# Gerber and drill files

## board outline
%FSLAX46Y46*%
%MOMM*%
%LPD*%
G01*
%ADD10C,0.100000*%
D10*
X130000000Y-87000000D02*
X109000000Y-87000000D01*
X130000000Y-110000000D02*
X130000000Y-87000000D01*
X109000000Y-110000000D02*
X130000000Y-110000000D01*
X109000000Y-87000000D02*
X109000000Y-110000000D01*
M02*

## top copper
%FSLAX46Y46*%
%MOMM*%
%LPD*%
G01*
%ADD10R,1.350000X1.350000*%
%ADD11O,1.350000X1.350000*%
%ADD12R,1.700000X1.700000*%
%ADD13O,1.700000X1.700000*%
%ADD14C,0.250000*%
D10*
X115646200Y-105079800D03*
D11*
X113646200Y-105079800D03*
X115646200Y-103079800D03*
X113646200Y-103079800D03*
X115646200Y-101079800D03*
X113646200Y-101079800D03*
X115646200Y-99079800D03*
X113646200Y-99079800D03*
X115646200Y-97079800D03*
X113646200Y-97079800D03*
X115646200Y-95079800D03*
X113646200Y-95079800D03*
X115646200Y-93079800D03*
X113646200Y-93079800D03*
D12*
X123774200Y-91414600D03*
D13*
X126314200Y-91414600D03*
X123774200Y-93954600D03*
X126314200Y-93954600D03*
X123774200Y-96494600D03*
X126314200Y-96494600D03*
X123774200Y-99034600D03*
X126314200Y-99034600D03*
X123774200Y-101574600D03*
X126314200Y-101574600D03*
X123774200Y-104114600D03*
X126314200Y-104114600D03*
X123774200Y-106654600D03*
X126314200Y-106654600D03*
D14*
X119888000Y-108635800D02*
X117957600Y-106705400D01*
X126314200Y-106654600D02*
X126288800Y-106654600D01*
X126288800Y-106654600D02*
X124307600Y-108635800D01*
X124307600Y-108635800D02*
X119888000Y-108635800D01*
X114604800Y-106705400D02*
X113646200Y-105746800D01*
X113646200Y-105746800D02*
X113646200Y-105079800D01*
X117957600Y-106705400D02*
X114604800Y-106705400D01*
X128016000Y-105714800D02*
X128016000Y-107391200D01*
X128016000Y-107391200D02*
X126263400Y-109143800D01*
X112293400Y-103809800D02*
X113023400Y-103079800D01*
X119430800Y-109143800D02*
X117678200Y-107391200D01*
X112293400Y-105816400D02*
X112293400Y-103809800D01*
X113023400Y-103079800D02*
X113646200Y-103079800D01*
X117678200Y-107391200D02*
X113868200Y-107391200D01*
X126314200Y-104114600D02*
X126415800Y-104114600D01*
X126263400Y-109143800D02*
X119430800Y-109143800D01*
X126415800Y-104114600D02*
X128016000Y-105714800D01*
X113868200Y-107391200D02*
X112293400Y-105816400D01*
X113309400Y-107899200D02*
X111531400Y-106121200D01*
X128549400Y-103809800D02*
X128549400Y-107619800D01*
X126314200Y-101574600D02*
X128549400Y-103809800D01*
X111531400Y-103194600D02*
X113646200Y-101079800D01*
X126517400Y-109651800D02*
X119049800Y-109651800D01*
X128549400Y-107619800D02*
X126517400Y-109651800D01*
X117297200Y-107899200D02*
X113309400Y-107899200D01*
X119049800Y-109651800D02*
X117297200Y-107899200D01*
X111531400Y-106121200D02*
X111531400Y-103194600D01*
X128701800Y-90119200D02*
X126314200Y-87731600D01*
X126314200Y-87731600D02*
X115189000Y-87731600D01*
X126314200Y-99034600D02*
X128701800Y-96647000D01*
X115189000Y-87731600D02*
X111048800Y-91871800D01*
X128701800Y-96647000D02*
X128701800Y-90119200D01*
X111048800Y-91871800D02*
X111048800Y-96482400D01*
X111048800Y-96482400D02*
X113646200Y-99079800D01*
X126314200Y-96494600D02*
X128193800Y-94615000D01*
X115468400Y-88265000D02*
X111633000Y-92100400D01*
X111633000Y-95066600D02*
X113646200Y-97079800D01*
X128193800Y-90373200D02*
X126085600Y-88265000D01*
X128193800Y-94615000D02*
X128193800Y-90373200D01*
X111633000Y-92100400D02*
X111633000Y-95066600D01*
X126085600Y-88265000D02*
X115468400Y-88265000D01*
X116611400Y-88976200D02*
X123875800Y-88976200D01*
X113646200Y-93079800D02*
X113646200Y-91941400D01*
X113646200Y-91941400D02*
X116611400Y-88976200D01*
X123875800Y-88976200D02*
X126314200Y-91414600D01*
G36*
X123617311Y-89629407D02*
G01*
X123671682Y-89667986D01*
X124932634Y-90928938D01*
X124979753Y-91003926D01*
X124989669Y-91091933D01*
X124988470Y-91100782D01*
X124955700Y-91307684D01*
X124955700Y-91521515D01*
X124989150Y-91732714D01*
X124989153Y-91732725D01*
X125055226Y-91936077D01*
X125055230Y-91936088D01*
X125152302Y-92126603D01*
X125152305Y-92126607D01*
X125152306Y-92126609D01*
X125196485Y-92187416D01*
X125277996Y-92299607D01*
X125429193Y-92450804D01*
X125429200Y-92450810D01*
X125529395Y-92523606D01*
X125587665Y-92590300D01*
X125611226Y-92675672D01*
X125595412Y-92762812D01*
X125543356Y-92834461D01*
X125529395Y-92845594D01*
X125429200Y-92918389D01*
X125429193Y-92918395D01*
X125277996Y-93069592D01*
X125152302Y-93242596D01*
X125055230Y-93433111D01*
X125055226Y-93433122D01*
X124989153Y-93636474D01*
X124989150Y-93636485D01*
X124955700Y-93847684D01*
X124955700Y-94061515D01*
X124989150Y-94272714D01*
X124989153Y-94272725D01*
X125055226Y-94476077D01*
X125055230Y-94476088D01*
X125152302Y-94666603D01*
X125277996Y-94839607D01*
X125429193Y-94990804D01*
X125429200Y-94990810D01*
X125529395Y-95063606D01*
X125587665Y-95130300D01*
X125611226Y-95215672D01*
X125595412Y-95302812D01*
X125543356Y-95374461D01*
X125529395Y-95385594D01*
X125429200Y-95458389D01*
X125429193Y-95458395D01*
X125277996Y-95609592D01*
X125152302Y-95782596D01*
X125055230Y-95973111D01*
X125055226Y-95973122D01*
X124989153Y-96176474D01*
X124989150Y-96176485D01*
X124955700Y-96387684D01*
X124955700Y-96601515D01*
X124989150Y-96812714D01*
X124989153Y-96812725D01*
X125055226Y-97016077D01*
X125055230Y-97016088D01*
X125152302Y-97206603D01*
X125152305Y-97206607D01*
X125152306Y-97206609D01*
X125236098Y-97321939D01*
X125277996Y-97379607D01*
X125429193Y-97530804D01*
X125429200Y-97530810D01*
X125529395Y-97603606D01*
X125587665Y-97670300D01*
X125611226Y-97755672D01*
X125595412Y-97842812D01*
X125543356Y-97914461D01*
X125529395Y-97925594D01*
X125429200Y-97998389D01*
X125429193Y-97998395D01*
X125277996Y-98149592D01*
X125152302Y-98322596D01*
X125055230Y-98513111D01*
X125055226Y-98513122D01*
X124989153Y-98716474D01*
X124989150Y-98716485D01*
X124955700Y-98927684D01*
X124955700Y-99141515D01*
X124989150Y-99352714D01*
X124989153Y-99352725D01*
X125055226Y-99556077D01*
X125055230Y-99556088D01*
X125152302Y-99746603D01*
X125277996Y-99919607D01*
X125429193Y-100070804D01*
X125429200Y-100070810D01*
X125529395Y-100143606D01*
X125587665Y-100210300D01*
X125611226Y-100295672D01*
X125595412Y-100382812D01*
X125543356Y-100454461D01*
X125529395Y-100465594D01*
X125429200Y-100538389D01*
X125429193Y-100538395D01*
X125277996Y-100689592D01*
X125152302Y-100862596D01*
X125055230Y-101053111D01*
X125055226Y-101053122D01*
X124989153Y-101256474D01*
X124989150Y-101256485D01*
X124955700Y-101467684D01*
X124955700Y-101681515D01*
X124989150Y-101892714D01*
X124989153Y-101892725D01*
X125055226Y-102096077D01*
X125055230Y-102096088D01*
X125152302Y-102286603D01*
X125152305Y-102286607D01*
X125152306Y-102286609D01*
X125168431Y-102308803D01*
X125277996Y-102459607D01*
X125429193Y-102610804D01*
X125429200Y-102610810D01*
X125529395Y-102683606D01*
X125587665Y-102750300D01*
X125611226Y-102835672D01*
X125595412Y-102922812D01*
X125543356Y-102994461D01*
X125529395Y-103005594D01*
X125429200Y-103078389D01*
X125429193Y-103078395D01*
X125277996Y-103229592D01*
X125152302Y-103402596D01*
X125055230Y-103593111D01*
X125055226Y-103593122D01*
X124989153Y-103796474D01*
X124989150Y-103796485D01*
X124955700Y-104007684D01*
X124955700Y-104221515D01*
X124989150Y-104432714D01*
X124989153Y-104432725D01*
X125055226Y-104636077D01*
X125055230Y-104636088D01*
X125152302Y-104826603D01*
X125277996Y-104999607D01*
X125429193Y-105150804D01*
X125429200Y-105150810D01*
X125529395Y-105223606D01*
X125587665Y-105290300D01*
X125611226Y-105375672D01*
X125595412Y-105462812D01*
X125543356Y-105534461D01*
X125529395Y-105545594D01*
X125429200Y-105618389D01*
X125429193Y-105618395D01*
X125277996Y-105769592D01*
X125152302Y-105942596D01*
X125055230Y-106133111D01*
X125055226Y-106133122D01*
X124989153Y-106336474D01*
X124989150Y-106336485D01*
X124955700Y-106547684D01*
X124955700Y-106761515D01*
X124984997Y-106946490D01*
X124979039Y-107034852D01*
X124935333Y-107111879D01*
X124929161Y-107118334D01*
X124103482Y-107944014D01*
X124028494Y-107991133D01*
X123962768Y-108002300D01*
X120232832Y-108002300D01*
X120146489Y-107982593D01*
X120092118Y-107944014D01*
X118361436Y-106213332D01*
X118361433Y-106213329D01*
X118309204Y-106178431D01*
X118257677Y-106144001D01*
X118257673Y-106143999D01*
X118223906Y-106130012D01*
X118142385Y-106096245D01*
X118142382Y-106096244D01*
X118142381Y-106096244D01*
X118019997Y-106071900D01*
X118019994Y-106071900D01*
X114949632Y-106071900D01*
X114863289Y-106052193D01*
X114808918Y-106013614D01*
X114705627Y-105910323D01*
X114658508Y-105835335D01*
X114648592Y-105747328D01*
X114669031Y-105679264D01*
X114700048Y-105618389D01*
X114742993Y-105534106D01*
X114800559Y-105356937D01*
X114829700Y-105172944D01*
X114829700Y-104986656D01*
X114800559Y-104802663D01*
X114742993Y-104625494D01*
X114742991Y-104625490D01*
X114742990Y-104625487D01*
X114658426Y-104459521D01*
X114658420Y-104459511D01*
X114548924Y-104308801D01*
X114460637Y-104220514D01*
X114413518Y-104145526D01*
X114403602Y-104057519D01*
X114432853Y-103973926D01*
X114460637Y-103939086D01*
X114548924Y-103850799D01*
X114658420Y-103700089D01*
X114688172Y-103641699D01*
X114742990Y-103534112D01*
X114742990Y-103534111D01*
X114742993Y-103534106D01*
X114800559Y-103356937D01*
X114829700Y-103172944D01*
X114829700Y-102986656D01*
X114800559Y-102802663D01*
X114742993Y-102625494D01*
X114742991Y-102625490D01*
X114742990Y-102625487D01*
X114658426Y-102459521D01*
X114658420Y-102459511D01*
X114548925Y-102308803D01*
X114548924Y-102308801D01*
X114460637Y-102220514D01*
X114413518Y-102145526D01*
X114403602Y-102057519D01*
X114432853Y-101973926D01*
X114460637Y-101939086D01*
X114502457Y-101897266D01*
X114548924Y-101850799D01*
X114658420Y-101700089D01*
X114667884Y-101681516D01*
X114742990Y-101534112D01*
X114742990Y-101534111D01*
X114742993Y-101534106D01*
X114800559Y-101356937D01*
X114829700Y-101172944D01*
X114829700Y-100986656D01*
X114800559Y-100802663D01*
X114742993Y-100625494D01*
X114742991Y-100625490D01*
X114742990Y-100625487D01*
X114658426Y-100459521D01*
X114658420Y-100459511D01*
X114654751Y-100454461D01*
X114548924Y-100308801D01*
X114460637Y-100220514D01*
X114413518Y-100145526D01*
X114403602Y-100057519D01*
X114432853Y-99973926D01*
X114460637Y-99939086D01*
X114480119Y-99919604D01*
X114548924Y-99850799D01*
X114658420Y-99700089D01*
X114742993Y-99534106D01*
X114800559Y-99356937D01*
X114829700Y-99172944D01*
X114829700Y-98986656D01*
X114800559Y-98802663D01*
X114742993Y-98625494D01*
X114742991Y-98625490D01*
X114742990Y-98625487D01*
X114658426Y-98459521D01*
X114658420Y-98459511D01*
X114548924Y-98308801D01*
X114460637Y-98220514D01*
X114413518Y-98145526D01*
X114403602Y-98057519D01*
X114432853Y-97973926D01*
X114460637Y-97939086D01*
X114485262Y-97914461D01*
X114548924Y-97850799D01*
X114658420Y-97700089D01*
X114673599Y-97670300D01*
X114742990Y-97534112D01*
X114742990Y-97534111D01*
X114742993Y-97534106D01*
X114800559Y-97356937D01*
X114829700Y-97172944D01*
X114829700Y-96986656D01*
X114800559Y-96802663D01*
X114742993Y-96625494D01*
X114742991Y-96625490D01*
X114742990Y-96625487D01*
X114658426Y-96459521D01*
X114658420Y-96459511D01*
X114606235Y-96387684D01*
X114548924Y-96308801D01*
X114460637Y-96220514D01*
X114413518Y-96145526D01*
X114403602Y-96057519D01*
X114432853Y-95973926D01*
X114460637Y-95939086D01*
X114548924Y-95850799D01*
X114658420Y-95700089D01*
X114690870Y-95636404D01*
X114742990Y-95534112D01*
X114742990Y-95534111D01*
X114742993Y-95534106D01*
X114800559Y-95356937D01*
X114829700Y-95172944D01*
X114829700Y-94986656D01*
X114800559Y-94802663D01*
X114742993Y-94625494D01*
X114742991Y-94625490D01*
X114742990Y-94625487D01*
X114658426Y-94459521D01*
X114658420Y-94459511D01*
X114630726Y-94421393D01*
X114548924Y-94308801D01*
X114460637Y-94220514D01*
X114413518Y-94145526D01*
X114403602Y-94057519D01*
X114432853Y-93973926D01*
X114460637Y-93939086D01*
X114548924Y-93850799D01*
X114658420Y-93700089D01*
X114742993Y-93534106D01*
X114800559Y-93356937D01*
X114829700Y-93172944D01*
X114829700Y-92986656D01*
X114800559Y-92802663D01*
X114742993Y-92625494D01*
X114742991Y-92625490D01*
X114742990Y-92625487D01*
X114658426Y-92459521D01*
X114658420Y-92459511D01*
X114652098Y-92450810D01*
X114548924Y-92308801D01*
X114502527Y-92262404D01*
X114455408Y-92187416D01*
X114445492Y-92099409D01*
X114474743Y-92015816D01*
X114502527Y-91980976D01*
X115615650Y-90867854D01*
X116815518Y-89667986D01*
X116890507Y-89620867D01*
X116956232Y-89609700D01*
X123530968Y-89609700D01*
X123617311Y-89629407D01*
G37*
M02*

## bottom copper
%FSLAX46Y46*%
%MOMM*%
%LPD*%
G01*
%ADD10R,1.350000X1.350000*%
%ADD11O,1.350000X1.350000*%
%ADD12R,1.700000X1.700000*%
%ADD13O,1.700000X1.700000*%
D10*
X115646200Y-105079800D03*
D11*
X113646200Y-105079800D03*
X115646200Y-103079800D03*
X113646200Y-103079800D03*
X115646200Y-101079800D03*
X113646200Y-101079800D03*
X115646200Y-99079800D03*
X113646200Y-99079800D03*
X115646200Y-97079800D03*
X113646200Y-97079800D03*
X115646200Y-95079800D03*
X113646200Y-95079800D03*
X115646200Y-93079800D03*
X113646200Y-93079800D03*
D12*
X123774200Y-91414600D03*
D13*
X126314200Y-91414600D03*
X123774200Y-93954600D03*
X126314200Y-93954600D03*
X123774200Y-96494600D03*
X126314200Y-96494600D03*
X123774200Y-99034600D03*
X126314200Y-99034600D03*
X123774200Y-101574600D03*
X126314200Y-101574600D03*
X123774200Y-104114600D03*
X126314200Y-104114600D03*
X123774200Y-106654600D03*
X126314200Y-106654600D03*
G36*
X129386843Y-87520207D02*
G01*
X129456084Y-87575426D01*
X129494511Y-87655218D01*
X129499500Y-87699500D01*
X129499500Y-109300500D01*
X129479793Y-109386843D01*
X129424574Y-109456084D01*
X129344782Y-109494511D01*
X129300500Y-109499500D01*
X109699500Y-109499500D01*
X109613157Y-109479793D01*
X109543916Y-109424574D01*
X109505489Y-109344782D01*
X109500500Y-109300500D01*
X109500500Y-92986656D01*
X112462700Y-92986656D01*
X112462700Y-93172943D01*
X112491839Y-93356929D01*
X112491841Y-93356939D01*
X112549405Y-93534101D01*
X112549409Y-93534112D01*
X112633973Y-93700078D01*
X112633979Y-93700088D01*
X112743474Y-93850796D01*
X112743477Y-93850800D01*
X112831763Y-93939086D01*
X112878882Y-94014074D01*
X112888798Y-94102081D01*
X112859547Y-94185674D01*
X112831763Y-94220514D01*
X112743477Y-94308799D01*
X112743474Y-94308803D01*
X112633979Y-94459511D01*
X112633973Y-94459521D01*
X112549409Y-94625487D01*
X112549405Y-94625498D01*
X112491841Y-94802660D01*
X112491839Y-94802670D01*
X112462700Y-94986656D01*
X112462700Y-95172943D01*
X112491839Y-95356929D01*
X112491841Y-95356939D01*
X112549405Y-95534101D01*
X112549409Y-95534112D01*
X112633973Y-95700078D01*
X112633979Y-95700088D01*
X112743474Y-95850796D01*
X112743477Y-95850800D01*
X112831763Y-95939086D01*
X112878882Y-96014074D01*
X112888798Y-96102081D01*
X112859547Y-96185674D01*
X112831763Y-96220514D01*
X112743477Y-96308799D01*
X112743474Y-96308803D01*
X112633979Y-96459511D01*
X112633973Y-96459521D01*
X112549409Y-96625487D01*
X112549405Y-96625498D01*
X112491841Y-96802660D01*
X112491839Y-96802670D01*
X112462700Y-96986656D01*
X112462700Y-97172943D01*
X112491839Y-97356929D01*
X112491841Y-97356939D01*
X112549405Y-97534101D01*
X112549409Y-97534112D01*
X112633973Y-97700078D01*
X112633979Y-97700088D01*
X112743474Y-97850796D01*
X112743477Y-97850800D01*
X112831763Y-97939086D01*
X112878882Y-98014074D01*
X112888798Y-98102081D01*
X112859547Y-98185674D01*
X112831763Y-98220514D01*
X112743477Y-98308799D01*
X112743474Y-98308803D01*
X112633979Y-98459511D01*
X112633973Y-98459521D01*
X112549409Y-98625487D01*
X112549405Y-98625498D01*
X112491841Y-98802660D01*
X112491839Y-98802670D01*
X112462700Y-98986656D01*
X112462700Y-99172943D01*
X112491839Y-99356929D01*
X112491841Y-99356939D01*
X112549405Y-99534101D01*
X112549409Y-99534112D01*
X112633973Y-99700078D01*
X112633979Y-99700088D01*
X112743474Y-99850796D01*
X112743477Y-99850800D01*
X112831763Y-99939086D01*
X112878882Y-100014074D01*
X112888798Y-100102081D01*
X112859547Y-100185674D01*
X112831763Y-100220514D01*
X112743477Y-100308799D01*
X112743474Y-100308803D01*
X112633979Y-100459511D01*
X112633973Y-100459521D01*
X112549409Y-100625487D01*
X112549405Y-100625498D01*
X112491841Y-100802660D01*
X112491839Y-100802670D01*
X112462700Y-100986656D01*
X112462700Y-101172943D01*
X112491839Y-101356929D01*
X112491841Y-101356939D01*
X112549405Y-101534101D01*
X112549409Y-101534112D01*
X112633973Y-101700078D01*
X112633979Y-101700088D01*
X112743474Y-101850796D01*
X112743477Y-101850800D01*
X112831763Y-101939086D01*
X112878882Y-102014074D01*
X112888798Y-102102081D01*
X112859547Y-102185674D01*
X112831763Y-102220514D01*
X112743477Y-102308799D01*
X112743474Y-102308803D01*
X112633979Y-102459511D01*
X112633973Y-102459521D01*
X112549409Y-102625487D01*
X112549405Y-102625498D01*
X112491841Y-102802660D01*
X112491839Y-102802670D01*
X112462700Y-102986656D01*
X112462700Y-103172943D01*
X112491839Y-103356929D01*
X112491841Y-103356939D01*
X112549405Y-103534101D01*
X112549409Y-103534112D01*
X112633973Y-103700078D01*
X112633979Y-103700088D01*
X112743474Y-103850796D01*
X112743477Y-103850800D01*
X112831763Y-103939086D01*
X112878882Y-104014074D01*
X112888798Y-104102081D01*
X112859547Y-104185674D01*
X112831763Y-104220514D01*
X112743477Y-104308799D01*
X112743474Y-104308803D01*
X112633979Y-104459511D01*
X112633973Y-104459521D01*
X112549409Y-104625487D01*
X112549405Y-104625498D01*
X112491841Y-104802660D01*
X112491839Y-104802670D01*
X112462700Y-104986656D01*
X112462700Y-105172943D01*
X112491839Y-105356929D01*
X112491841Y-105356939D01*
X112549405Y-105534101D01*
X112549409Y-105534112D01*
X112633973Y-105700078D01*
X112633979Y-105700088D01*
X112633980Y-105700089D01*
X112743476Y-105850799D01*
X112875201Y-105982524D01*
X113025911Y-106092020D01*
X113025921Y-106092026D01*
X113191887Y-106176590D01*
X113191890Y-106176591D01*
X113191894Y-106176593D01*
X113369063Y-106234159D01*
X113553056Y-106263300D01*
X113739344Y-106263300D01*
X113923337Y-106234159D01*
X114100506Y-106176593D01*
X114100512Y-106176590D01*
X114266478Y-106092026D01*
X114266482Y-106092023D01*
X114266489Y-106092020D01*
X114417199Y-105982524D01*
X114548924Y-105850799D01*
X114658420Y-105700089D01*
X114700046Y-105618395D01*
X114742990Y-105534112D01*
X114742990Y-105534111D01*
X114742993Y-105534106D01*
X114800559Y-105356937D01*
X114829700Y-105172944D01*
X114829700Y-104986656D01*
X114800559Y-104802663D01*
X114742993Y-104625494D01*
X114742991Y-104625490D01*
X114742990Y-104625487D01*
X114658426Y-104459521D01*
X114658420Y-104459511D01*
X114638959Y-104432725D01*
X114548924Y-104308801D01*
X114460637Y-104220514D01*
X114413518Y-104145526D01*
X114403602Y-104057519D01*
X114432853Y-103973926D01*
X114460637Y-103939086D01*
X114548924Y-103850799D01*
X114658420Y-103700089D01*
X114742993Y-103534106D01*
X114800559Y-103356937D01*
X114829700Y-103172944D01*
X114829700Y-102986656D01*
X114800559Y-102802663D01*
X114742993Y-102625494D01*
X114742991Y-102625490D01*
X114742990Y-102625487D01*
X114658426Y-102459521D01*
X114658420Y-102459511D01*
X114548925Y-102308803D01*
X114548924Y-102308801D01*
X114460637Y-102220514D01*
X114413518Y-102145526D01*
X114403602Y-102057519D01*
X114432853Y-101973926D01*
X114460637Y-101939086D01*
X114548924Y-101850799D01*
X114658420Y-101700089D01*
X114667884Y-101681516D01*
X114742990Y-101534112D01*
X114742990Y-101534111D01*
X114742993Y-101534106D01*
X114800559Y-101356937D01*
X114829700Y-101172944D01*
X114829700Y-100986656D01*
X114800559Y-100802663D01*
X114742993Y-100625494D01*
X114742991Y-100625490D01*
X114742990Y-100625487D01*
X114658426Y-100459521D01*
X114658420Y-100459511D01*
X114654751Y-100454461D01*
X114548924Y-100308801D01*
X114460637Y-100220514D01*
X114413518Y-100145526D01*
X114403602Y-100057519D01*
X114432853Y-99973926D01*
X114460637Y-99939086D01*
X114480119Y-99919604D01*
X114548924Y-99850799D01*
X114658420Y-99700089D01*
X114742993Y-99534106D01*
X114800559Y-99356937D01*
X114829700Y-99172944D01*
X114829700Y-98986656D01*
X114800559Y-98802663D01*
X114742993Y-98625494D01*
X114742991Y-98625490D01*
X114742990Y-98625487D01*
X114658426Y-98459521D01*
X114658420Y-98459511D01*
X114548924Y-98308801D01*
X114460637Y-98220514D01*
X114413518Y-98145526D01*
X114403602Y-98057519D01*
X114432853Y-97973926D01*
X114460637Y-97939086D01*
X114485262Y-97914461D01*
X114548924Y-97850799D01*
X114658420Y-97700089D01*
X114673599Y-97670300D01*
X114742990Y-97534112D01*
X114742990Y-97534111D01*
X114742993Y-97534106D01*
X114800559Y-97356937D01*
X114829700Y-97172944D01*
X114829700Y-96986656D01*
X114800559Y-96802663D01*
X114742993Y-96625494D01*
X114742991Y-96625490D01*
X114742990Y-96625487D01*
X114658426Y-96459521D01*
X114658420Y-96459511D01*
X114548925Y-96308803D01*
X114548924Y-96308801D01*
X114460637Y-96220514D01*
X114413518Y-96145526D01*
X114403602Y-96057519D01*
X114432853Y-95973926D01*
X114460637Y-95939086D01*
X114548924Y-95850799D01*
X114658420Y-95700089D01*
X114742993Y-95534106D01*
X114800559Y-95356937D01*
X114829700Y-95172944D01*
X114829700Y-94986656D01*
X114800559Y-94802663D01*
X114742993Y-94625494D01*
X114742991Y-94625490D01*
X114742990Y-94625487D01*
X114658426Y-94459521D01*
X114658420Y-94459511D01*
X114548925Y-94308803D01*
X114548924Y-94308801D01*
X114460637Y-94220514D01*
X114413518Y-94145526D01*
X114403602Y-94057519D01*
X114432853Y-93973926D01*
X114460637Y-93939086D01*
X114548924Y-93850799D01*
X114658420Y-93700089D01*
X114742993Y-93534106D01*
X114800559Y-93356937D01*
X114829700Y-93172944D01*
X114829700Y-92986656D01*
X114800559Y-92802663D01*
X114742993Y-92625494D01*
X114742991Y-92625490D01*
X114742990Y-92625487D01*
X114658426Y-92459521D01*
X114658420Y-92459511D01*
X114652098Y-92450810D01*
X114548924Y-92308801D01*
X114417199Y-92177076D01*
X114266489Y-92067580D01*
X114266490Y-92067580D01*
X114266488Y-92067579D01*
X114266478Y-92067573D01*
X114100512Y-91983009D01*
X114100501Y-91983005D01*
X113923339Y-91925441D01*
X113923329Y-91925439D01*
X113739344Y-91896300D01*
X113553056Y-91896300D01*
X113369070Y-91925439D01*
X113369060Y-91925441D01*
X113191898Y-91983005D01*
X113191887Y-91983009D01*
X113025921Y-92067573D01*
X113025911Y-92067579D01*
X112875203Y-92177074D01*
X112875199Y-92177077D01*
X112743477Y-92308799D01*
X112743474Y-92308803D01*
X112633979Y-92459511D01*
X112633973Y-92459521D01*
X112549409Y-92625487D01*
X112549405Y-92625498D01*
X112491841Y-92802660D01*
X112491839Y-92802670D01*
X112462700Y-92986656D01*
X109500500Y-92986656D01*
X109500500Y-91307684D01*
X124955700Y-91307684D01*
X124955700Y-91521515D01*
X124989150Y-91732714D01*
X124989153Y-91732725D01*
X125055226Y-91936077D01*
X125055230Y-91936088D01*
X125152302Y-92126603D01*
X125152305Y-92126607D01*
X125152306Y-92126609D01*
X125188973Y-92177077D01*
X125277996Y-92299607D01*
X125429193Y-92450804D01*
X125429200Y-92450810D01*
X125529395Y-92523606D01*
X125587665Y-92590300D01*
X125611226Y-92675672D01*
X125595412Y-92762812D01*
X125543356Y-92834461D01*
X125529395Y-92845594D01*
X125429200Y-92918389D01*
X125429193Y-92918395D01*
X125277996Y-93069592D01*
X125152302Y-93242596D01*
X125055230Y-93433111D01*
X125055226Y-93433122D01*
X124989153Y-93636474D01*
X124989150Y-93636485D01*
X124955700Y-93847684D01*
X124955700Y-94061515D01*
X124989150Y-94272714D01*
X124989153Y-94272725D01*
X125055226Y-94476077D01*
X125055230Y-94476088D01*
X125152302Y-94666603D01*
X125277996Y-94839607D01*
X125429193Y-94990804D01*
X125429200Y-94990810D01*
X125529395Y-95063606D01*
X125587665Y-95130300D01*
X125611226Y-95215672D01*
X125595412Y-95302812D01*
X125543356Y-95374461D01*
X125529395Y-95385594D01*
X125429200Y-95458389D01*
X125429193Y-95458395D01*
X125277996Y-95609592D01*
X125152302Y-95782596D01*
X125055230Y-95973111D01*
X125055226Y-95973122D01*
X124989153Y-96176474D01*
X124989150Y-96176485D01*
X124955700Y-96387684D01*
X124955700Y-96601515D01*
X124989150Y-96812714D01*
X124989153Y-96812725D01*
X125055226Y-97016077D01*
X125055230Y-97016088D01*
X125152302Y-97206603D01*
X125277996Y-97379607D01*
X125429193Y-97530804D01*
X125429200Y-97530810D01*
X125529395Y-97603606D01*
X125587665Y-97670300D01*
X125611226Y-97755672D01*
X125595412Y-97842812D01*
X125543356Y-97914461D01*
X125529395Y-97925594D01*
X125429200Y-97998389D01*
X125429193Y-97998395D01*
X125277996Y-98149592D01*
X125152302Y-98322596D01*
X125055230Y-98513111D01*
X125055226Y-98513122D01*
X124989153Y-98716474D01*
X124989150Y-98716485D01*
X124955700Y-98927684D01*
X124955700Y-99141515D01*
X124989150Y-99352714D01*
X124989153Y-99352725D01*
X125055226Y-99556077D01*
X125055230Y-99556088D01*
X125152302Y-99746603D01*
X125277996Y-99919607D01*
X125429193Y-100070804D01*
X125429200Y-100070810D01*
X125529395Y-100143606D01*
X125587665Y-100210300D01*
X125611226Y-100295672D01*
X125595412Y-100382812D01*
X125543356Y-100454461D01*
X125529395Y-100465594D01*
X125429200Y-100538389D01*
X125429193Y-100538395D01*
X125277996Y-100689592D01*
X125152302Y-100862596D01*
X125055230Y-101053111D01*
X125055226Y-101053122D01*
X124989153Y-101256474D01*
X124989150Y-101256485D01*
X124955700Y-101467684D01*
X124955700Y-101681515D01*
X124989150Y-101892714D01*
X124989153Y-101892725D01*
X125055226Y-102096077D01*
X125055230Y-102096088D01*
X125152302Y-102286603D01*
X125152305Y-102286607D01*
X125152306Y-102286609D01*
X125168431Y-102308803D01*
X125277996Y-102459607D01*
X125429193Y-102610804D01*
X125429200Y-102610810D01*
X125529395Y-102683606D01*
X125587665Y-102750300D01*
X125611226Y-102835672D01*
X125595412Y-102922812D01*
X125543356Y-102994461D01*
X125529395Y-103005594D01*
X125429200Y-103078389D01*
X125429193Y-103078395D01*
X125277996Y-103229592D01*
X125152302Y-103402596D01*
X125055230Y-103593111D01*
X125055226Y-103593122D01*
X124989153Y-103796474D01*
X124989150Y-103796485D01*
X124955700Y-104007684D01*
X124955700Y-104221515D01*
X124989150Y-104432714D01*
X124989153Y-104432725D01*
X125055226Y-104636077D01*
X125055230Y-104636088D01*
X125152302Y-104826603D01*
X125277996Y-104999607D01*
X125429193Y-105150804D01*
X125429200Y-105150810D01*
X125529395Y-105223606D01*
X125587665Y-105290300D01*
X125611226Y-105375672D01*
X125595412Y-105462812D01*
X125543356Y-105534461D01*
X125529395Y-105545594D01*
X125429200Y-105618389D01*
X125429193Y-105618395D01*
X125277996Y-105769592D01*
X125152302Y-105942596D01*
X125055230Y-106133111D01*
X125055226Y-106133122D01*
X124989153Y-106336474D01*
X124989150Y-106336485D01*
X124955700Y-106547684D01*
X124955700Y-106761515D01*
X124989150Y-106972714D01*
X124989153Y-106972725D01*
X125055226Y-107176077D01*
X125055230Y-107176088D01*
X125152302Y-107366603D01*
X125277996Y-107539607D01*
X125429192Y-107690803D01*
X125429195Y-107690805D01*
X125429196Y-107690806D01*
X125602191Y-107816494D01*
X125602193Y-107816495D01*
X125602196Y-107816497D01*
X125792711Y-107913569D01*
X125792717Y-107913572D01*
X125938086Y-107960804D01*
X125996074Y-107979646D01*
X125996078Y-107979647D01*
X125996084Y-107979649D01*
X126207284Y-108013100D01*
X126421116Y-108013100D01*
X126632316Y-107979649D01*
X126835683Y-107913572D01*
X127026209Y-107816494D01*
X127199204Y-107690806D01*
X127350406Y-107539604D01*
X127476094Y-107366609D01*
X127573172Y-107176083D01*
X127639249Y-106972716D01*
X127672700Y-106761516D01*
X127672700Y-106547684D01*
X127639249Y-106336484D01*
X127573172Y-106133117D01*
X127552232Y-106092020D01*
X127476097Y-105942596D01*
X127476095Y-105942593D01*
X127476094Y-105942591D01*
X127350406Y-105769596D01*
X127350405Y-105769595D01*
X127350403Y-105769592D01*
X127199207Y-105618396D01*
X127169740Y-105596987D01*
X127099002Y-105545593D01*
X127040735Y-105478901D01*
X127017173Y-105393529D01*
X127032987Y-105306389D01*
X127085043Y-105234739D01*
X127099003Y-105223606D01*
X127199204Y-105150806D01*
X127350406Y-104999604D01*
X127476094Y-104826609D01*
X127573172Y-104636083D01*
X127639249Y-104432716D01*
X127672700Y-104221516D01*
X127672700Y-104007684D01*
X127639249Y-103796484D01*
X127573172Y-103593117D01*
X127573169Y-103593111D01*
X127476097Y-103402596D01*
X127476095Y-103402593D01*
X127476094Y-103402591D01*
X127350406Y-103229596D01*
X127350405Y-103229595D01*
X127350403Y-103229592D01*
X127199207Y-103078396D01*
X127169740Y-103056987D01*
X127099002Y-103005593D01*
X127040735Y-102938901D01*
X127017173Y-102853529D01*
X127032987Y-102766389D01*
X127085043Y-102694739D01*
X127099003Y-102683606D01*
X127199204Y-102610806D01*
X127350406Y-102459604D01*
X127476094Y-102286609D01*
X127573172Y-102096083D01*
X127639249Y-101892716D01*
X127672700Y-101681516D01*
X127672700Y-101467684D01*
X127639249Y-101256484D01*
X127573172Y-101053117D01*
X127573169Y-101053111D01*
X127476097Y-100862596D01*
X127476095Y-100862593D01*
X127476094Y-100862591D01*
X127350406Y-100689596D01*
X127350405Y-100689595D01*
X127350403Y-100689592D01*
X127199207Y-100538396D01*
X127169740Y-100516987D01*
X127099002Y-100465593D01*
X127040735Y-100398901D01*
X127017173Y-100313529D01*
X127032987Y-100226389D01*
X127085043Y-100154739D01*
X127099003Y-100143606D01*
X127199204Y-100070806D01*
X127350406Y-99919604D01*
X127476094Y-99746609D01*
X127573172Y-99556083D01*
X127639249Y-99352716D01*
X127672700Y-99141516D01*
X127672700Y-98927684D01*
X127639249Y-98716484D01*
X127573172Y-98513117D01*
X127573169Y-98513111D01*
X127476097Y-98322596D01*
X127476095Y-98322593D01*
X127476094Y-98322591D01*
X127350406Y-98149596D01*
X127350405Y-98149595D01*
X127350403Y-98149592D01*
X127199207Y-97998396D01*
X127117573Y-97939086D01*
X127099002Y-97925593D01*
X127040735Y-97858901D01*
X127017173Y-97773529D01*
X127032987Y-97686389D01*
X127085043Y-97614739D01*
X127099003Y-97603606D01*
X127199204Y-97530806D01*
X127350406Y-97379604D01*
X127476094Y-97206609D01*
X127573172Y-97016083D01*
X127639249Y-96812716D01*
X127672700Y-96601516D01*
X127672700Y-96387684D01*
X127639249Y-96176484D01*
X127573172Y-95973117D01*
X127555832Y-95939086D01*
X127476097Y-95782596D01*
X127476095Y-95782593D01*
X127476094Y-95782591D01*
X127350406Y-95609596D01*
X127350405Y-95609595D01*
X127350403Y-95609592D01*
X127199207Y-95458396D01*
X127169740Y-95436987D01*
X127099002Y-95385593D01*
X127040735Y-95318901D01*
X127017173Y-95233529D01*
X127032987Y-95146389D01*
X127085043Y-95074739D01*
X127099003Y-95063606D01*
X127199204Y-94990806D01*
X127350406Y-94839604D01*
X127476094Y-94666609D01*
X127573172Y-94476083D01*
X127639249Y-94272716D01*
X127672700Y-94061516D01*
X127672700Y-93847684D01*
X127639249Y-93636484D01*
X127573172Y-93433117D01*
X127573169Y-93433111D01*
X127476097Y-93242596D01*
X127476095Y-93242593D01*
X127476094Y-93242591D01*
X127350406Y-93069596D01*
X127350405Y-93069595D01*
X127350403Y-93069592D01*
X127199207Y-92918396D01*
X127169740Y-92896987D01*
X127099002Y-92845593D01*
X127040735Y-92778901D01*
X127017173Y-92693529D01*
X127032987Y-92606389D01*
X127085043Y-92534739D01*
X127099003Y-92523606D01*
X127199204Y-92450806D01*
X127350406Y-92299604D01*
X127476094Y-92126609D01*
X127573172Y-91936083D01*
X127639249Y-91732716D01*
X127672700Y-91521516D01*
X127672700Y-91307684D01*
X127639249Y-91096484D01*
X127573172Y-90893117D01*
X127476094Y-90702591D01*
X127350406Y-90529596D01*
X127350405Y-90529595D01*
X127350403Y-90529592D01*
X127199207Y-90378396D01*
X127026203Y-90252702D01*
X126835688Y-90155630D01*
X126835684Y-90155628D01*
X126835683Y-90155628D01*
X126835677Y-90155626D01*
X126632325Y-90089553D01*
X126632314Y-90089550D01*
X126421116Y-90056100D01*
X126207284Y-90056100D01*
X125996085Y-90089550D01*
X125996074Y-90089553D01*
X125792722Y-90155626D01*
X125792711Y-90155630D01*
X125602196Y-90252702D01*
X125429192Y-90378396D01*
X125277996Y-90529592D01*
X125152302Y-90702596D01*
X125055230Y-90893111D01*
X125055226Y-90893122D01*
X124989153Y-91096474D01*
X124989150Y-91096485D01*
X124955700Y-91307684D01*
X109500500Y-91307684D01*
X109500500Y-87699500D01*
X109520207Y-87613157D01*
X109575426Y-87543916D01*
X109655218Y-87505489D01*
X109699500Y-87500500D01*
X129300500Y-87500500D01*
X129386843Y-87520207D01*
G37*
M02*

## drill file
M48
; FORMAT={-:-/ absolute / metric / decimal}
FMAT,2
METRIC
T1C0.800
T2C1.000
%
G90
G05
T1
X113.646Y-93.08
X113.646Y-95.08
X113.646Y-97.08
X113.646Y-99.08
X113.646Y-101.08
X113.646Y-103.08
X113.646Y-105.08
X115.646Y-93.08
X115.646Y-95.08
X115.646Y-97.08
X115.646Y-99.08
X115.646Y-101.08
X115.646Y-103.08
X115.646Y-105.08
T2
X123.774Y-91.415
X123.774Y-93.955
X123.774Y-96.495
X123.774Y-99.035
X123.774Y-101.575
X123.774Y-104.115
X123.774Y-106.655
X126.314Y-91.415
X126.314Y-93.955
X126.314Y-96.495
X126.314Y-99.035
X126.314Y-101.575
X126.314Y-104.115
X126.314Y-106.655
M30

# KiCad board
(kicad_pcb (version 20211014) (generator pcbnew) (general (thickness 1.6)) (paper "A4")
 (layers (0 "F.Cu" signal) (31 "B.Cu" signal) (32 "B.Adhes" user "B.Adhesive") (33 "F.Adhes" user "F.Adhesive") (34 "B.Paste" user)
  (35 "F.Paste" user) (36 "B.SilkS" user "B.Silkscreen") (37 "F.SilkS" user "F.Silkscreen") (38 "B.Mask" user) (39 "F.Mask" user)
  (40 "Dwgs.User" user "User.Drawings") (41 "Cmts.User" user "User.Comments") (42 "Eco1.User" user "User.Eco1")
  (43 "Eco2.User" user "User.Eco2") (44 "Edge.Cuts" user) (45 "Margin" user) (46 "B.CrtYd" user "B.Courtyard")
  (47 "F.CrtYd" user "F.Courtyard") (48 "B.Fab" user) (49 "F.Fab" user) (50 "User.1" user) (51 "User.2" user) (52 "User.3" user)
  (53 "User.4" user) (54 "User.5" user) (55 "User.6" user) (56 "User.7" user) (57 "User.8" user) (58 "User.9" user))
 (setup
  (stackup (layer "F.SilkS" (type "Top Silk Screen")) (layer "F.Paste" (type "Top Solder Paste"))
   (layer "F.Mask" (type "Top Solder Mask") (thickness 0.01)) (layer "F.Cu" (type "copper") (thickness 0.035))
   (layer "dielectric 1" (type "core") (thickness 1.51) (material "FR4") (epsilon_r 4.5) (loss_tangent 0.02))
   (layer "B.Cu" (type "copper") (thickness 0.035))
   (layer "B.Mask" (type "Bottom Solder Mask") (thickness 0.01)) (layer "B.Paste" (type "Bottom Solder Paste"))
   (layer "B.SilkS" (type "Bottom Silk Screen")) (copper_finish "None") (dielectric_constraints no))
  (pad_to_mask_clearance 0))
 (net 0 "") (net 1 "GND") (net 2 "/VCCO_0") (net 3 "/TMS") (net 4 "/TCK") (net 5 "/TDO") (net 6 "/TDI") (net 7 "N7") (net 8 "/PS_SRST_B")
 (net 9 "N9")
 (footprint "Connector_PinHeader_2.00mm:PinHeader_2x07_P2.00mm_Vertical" (layer "F.Cu") (at 115.6462 105.0798 180)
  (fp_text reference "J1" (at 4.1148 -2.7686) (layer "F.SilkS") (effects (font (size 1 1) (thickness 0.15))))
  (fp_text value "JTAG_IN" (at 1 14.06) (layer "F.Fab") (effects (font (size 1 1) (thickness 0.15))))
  (pad "1" thru_hole rect (at 0 0 180) (size 1.35 1.35) (drill 0.8) (layers *.Cu *.Mask) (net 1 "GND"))
  (pad "2" thru_hole oval (at 2 0 180) (size 1.35 1.35) (drill 0.8) (layers *.Cu *.Mask) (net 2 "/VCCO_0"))
  (pad "3" thru_hole oval (at 0 2 180) (size 1.35 1.35) (drill 0.8) (layers *.Cu *.Mask) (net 1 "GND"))
  (pad "4" thru_hole oval (at 2 2 180) (size 1.35 1.35) (drill 0.8) (layers *.Cu *.Mask) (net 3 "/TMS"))
  (pad "5" thru_hole oval (at 0 4 180) (size 1.35 1.35) (drill 0.8) (layers *.Cu *.Mask) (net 1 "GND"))
  (pad "6" thru_hole oval (at 2 4 180) (size 1.35 1.35) (drill 0.8) (layers *.Cu *.Mask) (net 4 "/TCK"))
  (pad "7" thru_hole oval (at 0 6 180) (size 1.35 1.35) (drill 0.8) (layers *.Cu *.Mask) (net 1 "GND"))
  (pad "8" thru_hole oval (at 2 6 180) (size 1.35 1.35) (drill 0.8) (layers *.Cu *.Mask) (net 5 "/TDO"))
  (pad "9" thru_hole oval (at 0 8 180) (size 1.35 1.35) (drill 0.8) (layers *.Cu *.Mask) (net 1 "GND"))
  (pad "10" thru_hole oval (at 2 8 180) (size 1.35 1.35) (drill 0.8) (layers *.Cu *.Mask) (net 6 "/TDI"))
  (pad "11" thru_hole oval (at 0 10 180) (size 1.35 1.35) (drill 0.8) (layers *.Cu *.Mask) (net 1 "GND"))
  (pad "12" thru_hole oval (at 2 10 180) (size 1.35 1.35) (drill 0.8) (layers *.Cu *.Mask) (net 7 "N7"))
  (pad "13" thru_hole oval (at 0 12 180) (size 1.35 1.35) (drill 0.8) (layers *.Cu *.Mask) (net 1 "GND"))
  (pad "14" thru_hole oval (at 2 12 180) (size 1.35 1.35) (drill 0.8) (layers *.Cu *.Mask) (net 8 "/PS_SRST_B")))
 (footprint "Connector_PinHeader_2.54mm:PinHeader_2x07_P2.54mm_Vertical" (layer "F.Cu") (at 123.7742 91.4146)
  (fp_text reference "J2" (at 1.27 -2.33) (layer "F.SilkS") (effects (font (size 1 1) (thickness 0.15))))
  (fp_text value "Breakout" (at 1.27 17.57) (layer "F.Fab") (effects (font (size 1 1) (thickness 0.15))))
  (pad "1" thru_hole rect (at 0 0) (size 1.7 1.7) (drill 1) (layers *.Cu *.Mask) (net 1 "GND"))
  (pad "2" thru_hole oval (at 2.54 0) (size 1.7 1.7) (drill 1) (layers *.Cu *.Mask) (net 8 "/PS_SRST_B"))
  (pad "3" thru_hole oval (at 0 2.54) (size 1.7 1.7) (drill 1) (layers *.Cu *.Mask) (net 1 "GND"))
  (pad "4" thru_hole oval (at 2.54 2.54) (size 1.7 1.7) (drill 1) (layers *.Cu *.Mask) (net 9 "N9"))
  (pad "5" thru_hole oval (at 0 5.08) (size 1.7 1.7) (drill 1) (layers *.Cu *.Mask) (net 1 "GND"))
  (pad "6" thru_hole oval (at 2.54 5.08) (size 1.7 1.7) (drill 1) (layers *.Cu *.Mask) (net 6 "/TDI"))
  (pad "7" thru_hole oval (at 0 7.62) (size 1.7 1.7) (drill 1) (layers *.Cu *.Mask) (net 1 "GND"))
  (pad "8" thru_hole oval (at 2.54 7.62) (size 1.7 1.7) (drill 1) (layers *.Cu *.Mask) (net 5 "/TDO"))
  (pad "9" thru_hole oval (at 0 10.16) (size 1.7 1.7) (drill 1) (layers *.Cu *.Mask) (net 1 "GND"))
  (pad "10" thru_hole oval (at 2.54 10.16) (size 1.7 1.7) (drill 1) (layers *.Cu *.Mask) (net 4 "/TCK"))
  (pad "11" thru_hole oval (at 0 12.7) (size 1.7 1.7) (drill 1) (layers *.Cu *.Mask) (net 1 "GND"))
  (pad "12" thru_hole oval (at 2.54 12.7) (size 1.7 1.7) (drill 1) (layers *.Cu *.Mask) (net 3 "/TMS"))
  (pad "13" thru_hole oval (at 0 15.24) (size 1.7 1.7) (drill 1) (layers *.Cu *.Mask) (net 1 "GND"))
  (pad "14" thru_hole oval (at 2.54 15.24) (size 1.7 1.7) (drill 1) (layers *.Cu *.Mask) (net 2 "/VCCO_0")))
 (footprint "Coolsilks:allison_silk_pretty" (layer "B.Cu") (at 119.507 104.7496 180)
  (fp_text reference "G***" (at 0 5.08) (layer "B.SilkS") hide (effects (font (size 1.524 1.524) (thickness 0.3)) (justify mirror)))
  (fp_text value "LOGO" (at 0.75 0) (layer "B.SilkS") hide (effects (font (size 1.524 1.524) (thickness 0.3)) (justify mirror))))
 (gr_line (start 130 87) (end 109 87) (layer "Edge.Cuts") (width 0.1))
 (gr_line (start 130 110) (end 130 87) (layer "Edge.Cuts") (width 0.1))
 (gr_line (start 109 110) (end 130 110) (layer "Edge.Cuts") (width 0.1))
 (gr_line (start 109 87) (end 109 110) (layer "Edge.Cuts") (width 0.1))
 (segment (start 119.888 108.6358) (end 117.9576 106.7054) (width 0.25) (layer "F.Cu") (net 2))
 (segment (start 126.3142 106.6546) (end 126.2888 106.6546) (width 0.25) (layer "F.Cu") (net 2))
 (segment (start 126.2888 106.6546) (end 124.3076 108.6358) (width 0.25) (layer "F.Cu") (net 2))
 (segment (start 124.3076 108.6358) (end 119.888 108.6358) (width 0.25) (layer "F.Cu") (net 2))
 (segment (start 114.6048 106.7054) (end 113.6462 105.7468) (width 0.25) (layer "F.Cu") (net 2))
 (segment (start 113.6462 105.7468) (end 113.6462 105.0798) (width 0.25) (layer "F.Cu") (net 2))
 (segment (start 117.9576 106.7054) (end 114.6048 106.7054) (width 0.25) (layer "F.Cu") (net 2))
 (segment (start 128.016 105.7148) (end 128.016 107.3912) (width 0.25) (layer "F.Cu") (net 3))
 (segment (start 128.016 107.3912) (end 126.2634 109.1438) (width 0.25) (layer "F.Cu") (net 3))
 (segment (start 112.2934 103.8098) (end 113.0234 103.0798) (width 0.25) (layer "F.Cu") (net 3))
 (segment (start 119.4308 109.1438) (end 117.6782 107.3912) (width 0.25) (layer "F.Cu") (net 3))
 (segment (start 112.2934 105.8164) (end 112.2934 103.8098) (width 0.25) (layer "F.Cu") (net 3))
 (segment (start 113.0234 103.0798) (end 113.6462 103.0798) (width 0.25) (layer "F.Cu") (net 3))
 (segment (start 117.6782 107.3912) (end 113.8682 107.3912) (width 0.25) (layer "F.Cu") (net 3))
 (segment (start 126.3142 104.1146) (end 126.4158 104.1146) (width 0.25) (layer "F.Cu") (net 3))
 (segment (start 126.2634 109.1438) (end 119.4308 109.1438) (width 0.25) (layer "F.Cu") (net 3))
 (segment (start 126.4158 104.1146) (end 128.016 105.7148) (width 0.25) (layer "F.Cu") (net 3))
 (segment (start 113.8682 107.3912) (end 112.2934 105.8164) (width 0.25) (layer "F.Cu") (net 3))
 (segment (start 113.3094 107.8992) (end 111.5314 106.1212) (width 0.25) (layer "F.Cu") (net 4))
 (segment (start 128.5494 103.8098) (end 128.5494 107.6198) (width 0.25) (layer "F.Cu") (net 4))
 (segment (start 126.3142 101.5746) (end 128.5494 103.8098) (width 0.25) (layer "F.Cu") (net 4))
 (segment (start 111.5314 103.1946) (end 113.6462 101.0798) (width 0.25) (layer "F.Cu") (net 4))
 (segment (start 126.5174 109.6518) (end 119.0498 109.6518) (width 0.25) (layer "F.Cu") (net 4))
 (segment (start 128.5494 107.6198) (end 126.5174 109.6518) (width 0.25) (layer "F.Cu") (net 4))
 (segment (start 117.2972 107.8992) (end 113.3094 107.8992) (width 0.25) (layer "F.Cu") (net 4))
 (segment (start 119.0498 109.6518) (end 117.2972 107.8992) (width 0.25) (layer "F.Cu") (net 4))
 (segment (start 111.5314 106.1212) (end 111.5314 103.1946) (width 0.25) (layer "F.Cu") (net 4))
 (segment (start 128.7018 90.1192) (end 126.3142 87.7316) (width 0.25) (layer "F.Cu") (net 5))
 (segment (start 126.3142 87.7316) (end 115.189 87.7316) (width 0.25) (layer "F.Cu") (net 5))
 (segment (start 126.3142 99.0346) (end 128.7018 96.647) (width 0.25) (layer "F.Cu") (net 5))
 (segment (start 115.189 87.7316) (end 111.0488 91.8718) (width 0.25) (layer "F.Cu") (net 5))
 (segment (start 128.7018 96.647) (end 128.7018 90.1192) (width 0.25) (layer "F.Cu") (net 5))
 (segment (start 111.0488 91.8718) (end 111.0488 96.4824) (width 0.25) (layer "F.Cu") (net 5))
 (segment (start 111.0488 96.4824) (end 113.6462 99.0798) (width 0.25) (layer "F.Cu") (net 5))
 (segment (start 126.3142 96.4946) (end 128.1938 94.615) (width 0.25) (layer "F.Cu") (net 6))
 (segment (start 115.4684 88.265) (end 111.633 92.1004) (width 0.25) (layer "F.Cu") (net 6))
 (segment (start 111.633 95.0666) (end 113.6462 97.0798) (width 0.25) (layer "F.Cu") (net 6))
 (segment (start 128.1938 90.3732) (end 126.0856 88.265) (width 0.25) (layer "F.Cu") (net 6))
 (segment (start 128.1938 94.615) (end 128.1938 90.3732) (width 0.25) (layer "F.Cu") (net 6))
 (segment (start 111.633 92.1004) (end 111.633 95.0666) (width 0.25) (layer "F.Cu") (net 6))
 (segment (start 126.0856 88.265) (end 115.4684 88.265) (width 0.25) (layer "F.Cu") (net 6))
 (segment (start 116.6114 88.9762) (end 123.8758 88.9762) (width 0.25) (layer "F.Cu") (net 8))
 (segment (start 113.6462 93.0798) (end 113.6462 91.9414) (width 0.25) (layer "F.Cu") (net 8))
 (segment (start 113.6462 91.9414) (end 116.6114 88.9762) (width 0.25) (layer "F.Cu") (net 8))
 (segment (start 123.8758 88.9762) (end 126.3142 91.4146) (width 0.25) (layer "F.Cu") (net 8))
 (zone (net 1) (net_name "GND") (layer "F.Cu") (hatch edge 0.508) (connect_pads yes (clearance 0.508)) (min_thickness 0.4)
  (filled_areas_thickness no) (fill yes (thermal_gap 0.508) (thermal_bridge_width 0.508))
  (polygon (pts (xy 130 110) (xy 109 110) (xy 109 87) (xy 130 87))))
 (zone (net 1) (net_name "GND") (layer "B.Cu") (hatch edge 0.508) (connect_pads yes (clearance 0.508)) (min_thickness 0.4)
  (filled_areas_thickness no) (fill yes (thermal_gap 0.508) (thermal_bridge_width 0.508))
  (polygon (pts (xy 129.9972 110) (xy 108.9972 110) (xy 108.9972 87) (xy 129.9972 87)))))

